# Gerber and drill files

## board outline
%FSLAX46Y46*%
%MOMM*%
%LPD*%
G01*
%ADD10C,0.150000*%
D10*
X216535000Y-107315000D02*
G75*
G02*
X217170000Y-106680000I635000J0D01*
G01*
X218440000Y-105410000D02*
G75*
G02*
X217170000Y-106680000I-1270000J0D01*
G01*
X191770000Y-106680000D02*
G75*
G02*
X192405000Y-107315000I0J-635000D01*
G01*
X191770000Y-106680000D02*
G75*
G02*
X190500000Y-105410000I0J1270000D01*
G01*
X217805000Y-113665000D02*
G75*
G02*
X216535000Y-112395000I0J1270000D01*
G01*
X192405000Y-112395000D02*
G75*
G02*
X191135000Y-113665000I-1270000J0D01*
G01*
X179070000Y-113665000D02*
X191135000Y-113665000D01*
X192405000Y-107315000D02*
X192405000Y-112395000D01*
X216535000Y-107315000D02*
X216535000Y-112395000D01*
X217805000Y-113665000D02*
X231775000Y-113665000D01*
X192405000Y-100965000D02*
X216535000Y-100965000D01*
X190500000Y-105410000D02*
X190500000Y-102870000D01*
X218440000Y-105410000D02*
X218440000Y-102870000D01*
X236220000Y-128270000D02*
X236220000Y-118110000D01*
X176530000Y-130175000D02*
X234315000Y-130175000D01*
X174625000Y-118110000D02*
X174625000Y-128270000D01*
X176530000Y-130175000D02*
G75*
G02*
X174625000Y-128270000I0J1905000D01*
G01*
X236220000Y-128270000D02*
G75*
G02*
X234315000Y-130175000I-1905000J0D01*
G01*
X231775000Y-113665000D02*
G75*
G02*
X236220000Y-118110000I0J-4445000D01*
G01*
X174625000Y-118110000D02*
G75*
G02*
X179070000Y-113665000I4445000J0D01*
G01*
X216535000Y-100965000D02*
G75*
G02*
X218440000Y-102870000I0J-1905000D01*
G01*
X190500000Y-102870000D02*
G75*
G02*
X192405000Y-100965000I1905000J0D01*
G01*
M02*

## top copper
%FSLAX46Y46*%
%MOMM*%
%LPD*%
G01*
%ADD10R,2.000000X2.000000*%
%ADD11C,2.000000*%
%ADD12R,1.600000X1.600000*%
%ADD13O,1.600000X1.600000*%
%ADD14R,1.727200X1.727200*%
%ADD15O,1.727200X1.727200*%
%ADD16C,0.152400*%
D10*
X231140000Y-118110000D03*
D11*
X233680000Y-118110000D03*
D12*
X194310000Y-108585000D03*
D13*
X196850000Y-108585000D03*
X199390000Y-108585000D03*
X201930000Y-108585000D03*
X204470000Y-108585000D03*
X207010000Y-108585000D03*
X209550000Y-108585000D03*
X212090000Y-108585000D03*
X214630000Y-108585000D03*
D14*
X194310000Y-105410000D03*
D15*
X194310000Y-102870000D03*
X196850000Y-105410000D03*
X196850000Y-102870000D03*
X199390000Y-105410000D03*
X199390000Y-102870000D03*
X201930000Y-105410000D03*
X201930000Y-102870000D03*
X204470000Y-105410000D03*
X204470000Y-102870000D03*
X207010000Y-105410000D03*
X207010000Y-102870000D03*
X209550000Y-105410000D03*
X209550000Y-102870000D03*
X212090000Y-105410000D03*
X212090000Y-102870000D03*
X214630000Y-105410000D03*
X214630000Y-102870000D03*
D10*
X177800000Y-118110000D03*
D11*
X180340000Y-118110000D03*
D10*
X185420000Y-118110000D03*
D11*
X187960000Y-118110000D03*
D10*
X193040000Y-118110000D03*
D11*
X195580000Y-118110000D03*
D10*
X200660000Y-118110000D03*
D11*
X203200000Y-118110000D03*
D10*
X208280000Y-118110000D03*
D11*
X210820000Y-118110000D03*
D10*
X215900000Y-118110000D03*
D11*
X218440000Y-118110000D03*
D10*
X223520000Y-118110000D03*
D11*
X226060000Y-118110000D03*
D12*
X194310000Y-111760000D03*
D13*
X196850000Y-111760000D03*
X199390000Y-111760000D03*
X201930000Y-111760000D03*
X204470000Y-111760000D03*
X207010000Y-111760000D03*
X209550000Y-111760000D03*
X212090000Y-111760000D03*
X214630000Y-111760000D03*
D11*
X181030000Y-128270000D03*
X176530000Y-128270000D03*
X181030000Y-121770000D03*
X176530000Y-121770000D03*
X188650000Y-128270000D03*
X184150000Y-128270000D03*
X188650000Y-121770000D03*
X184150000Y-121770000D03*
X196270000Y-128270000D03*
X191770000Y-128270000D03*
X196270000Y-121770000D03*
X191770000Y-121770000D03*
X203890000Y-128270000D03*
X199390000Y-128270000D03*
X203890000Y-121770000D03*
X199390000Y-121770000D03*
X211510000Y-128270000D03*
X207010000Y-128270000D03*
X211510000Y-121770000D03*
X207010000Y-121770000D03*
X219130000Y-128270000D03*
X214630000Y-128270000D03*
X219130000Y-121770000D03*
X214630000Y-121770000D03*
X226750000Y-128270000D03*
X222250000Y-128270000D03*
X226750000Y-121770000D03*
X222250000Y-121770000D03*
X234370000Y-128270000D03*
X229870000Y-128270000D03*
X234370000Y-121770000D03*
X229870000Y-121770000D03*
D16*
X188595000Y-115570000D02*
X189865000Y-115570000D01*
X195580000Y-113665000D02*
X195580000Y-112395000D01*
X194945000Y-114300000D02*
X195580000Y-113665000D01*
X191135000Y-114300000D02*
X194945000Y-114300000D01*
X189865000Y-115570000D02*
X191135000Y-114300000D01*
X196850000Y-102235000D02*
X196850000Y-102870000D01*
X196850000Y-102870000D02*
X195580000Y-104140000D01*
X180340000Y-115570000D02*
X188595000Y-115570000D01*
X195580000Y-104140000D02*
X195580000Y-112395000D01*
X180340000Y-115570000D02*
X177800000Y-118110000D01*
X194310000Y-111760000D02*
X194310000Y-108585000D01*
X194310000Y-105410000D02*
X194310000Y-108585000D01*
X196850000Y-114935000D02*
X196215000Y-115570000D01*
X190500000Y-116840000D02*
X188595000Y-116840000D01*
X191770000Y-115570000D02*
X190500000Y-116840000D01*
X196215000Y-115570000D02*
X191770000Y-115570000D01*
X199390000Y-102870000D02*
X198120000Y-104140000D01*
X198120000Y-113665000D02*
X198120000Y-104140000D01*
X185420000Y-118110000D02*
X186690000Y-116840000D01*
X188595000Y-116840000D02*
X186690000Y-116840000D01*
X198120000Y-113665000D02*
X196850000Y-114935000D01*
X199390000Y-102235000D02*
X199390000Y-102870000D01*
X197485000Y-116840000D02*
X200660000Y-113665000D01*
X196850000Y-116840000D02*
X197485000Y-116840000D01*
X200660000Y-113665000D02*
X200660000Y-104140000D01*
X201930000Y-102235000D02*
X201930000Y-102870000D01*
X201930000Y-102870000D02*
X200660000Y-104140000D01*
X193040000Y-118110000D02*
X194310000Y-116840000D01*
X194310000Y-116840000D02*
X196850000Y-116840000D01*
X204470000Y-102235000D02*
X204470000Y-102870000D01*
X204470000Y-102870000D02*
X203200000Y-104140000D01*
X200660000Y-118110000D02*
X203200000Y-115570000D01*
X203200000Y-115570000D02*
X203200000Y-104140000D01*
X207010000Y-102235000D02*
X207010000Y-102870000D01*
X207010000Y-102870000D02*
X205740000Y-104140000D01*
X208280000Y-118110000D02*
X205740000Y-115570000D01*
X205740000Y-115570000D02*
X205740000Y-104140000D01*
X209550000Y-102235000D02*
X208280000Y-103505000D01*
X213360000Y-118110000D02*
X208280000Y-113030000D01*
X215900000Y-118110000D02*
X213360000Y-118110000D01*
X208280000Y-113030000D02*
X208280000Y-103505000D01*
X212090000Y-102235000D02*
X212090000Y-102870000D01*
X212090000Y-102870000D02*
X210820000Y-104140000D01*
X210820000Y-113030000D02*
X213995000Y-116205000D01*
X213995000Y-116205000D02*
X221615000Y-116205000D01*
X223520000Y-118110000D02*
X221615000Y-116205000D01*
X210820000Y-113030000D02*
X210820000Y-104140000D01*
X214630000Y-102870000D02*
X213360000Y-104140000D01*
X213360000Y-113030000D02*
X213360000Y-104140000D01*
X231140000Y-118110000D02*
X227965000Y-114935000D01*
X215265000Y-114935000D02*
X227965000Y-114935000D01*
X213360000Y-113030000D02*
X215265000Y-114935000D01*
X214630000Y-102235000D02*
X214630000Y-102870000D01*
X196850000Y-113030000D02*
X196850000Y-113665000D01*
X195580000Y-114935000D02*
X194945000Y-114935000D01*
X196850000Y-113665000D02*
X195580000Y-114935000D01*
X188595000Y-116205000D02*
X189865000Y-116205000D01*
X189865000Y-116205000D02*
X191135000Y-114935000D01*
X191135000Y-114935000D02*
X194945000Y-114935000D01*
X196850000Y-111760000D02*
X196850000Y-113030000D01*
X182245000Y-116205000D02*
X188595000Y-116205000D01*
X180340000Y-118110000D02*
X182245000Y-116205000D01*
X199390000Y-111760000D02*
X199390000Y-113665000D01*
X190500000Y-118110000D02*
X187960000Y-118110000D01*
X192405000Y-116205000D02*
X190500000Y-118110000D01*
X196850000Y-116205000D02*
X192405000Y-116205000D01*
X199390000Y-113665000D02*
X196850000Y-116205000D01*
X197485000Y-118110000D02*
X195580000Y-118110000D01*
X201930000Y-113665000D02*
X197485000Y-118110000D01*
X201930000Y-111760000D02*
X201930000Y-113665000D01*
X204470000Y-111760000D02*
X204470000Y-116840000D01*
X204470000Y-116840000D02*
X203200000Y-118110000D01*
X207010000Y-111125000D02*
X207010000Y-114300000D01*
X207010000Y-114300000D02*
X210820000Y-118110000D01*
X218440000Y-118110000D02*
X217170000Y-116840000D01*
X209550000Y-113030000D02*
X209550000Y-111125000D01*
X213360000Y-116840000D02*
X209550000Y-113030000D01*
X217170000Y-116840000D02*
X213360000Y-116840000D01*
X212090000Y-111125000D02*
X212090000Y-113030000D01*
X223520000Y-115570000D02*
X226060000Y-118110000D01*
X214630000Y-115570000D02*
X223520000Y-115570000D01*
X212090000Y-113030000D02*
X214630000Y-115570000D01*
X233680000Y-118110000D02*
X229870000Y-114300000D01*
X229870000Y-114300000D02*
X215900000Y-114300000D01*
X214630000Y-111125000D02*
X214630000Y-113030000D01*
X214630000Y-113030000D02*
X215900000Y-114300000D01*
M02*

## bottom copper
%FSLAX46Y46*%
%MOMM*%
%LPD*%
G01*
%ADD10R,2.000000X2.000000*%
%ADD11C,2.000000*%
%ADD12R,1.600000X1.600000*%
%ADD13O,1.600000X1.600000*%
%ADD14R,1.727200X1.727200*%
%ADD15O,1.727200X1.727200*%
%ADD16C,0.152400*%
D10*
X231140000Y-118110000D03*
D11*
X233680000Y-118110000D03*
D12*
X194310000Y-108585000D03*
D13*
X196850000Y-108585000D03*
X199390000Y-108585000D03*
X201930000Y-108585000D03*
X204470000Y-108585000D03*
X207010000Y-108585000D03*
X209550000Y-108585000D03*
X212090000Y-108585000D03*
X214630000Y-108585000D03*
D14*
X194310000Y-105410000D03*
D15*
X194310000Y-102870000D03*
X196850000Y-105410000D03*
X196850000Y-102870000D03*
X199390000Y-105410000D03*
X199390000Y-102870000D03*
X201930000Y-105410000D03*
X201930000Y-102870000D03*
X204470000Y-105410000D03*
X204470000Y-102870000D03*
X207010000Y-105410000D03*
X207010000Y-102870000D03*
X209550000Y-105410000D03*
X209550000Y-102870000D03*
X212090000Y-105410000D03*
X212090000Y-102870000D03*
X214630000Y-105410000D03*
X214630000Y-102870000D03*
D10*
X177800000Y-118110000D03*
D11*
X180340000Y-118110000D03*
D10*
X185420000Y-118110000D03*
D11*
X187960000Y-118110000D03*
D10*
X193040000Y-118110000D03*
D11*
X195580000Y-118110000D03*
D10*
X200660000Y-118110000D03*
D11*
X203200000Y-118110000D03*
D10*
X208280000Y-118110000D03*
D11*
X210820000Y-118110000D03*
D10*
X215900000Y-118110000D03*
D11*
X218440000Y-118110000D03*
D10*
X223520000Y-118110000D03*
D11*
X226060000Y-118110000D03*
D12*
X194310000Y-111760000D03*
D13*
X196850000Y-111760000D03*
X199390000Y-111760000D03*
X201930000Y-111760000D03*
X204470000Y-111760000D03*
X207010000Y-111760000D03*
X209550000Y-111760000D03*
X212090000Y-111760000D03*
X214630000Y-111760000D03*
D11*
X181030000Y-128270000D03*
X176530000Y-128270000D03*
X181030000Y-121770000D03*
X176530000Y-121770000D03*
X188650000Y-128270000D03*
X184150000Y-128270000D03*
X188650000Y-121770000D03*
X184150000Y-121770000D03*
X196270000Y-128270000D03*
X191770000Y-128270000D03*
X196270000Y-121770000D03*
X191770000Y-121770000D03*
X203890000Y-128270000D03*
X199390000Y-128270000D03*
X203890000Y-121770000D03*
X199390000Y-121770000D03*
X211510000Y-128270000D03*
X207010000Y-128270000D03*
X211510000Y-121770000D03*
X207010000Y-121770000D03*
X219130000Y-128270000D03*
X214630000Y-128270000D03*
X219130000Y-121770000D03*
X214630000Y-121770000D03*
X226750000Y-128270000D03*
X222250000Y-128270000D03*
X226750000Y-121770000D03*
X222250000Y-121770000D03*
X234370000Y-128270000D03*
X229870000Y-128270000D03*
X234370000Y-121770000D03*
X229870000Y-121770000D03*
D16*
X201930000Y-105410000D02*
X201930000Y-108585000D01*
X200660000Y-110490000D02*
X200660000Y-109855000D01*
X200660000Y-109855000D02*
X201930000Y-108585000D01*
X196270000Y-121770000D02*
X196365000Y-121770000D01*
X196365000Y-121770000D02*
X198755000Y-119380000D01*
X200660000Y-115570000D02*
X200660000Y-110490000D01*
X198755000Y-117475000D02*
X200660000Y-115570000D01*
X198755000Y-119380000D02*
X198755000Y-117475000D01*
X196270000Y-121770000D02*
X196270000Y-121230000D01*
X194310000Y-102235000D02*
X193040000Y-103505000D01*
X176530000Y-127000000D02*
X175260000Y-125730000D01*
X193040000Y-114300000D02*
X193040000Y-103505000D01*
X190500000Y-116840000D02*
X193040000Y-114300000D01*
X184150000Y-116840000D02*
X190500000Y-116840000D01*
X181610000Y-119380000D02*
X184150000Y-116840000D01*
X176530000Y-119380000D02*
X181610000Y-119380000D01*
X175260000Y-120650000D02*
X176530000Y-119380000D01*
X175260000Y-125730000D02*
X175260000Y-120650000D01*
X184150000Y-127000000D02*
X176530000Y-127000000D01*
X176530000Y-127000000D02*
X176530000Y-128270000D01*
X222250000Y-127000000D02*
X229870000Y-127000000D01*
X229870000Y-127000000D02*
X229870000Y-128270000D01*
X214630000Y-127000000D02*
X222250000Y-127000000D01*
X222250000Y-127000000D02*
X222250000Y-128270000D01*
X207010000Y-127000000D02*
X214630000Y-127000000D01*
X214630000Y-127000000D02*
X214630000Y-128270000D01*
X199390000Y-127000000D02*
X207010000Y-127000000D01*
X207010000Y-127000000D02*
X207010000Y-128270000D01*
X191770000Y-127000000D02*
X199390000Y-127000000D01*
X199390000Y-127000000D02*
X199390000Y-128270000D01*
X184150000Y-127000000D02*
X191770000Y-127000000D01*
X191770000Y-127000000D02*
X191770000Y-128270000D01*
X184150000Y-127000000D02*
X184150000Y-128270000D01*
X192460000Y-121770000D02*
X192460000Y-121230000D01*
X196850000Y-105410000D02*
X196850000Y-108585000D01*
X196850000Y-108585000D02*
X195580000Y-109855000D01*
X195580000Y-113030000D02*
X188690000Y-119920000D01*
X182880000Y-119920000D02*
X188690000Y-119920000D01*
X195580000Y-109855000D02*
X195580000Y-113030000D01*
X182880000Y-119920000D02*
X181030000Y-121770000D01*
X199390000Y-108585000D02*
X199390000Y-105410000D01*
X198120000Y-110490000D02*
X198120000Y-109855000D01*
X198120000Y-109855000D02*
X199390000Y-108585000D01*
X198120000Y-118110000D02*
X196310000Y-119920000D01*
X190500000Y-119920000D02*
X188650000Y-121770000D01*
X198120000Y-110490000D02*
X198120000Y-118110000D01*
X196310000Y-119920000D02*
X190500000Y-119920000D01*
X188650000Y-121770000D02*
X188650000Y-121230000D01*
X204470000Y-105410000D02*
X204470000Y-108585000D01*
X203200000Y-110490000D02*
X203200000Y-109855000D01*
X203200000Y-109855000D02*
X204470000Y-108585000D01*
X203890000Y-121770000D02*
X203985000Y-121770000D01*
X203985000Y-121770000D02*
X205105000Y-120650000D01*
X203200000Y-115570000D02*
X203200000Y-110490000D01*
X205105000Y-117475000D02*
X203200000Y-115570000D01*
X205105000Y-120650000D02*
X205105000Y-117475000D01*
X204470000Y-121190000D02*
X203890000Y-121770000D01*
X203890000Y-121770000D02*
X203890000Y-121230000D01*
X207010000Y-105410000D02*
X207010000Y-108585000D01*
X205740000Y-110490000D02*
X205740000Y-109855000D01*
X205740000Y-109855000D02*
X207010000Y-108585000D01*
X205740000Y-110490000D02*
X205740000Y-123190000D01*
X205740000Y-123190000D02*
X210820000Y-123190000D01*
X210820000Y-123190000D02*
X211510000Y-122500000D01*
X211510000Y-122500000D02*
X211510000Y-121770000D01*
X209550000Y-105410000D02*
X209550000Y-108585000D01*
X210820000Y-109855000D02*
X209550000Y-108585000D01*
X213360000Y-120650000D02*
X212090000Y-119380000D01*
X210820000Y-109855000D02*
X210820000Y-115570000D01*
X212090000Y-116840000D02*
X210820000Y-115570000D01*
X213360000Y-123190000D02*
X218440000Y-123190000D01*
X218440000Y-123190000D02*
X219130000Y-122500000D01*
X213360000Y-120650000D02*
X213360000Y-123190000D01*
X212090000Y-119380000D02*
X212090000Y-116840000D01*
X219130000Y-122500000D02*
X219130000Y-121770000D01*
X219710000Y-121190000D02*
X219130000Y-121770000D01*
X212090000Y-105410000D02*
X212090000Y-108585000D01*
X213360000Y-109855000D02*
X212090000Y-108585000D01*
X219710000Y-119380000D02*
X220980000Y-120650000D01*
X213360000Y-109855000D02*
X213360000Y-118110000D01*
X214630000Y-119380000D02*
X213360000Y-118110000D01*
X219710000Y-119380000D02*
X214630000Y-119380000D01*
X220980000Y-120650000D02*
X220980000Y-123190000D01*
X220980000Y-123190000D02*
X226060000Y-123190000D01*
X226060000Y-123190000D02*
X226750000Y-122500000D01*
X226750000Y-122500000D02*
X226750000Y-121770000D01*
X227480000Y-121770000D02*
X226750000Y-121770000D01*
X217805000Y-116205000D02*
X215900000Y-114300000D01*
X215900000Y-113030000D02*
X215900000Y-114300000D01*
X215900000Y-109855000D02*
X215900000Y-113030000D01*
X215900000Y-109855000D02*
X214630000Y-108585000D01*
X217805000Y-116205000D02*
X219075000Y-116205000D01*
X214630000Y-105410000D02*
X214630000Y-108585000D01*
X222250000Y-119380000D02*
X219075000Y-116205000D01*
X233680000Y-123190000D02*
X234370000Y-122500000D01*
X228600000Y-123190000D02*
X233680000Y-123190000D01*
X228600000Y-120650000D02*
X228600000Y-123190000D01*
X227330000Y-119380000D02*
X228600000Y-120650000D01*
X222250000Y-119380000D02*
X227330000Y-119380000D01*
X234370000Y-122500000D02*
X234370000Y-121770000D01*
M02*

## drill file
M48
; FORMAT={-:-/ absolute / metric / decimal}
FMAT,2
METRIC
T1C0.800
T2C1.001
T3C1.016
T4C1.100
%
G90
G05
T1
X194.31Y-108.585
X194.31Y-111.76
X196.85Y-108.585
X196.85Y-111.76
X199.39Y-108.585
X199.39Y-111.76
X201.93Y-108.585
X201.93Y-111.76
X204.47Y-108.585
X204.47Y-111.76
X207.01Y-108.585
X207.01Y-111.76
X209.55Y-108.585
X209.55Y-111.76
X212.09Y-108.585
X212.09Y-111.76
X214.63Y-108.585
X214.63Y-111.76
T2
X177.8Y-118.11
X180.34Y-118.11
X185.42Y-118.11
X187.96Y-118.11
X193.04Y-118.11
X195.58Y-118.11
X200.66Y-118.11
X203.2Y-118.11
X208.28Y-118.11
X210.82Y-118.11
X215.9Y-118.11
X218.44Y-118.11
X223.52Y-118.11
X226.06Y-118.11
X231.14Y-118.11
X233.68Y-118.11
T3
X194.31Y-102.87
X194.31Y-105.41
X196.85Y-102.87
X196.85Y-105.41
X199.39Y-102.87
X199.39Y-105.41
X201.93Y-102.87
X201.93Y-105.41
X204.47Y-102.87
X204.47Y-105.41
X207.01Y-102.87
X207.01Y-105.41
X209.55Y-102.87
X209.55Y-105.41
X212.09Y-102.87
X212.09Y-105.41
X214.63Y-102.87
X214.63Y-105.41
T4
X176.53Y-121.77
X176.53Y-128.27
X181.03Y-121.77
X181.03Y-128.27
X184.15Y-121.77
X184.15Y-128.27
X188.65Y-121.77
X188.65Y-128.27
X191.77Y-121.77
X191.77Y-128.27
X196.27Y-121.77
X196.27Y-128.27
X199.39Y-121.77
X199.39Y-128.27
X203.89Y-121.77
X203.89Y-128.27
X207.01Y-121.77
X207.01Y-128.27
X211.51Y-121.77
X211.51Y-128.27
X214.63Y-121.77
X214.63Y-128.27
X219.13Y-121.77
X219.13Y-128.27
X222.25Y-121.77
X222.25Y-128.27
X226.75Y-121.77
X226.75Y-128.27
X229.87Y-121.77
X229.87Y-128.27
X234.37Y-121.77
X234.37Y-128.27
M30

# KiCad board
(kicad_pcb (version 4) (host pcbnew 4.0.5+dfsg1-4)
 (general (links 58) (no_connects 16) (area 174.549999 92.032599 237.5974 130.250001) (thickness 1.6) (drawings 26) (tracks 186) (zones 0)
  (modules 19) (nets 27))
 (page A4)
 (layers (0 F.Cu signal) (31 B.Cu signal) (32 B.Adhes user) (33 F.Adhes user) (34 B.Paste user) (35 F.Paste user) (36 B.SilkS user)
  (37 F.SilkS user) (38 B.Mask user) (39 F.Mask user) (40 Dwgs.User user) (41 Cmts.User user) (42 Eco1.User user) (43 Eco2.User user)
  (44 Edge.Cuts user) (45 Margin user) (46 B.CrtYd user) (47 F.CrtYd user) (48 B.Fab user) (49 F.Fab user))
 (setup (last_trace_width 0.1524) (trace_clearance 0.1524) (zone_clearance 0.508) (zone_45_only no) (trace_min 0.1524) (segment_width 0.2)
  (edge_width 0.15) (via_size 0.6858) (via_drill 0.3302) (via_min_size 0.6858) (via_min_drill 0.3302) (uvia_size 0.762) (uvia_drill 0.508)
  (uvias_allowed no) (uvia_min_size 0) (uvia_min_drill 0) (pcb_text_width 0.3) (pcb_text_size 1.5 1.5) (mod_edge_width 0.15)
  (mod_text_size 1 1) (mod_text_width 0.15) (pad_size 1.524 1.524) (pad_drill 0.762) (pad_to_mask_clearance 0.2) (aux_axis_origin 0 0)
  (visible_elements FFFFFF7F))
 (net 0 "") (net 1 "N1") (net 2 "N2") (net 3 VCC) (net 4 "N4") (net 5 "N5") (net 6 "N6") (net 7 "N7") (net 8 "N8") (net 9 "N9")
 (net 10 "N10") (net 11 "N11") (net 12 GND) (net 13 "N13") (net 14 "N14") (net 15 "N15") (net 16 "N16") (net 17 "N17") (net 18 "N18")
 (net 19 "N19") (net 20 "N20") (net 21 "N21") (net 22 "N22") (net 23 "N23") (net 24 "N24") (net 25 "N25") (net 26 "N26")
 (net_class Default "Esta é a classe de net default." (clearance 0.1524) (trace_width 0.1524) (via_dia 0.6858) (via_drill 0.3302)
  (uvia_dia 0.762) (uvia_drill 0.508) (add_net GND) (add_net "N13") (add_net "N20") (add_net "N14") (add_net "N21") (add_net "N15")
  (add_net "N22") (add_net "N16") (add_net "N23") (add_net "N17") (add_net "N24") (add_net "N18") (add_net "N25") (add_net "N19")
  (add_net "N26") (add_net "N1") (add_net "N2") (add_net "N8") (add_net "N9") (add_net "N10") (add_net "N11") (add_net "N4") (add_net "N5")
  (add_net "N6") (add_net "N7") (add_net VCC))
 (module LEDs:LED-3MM (layer F.Cu) (at 231.14 118.11)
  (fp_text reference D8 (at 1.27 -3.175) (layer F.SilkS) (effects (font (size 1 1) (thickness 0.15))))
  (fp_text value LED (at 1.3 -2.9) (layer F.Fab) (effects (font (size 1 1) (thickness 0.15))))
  (pad 1 thru_hole rect (at 0 0 90) (size 2 2) (drill 1.00076) (layers *.Cu *.Mask) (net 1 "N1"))
  (pad 2 thru_hole circle (at 2.54 0) (size 2 2) (drill 1.00076) (layers *.Cu *.Mask) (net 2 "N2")))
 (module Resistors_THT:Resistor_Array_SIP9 (layer F.Cu) (at 194.31 108.585)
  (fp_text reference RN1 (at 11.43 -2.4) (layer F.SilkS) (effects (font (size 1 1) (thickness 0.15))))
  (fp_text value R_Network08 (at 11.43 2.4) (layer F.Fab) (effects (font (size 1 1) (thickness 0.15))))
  (pad 1 thru_hole rect (at 0 0) (size 1.6 1.6) (drill 0.8) (layers *.Cu *.Mask) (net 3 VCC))
  (pad 2 thru_hole oval (at 2.54 0) (size 1.6 1.6) (drill 0.8) (layers *.Cu *.Mask) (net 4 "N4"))
  (pad 3 thru_hole oval (at 5.08 0) (size 1.6 1.6) (drill 0.8) (layers *.Cu *.Mask) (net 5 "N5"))
  (pad 4 thru_hole oval (at 7.62 0) (size 1.6 1.6) (drill 0.8) (layers *.Cu *.Mask) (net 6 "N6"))
  (pad 5 thru_hole oval (at 10.16 0) (size 1.6 1.6) (drill 0.8) (layers *.Cu *.Mask) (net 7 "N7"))
  (pad 6 thru_hole oval (at 12.7 0) (size 1.6 1.6) (drill 0.8) (layers *.Cu *.Mask) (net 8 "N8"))
  (pad 7 thru_hole oval (at 15.24 0) (size 1.6 1.6) (drill 0.8) (layers *.Cu *.Mask) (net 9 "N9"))
  (pad 8 thru_hole oval (at 17.78 0) (size 1.6 1.6) (drill 0.8) (layers *.Cu *.Mask) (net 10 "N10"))
  (pad 9 thru_hole oval (at 20.32 0) (size 1.6 1.6) (drill 0.8) (layers *.Cu *.Mask) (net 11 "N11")))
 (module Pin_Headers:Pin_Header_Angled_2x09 (layer F.Cu) (at 194.31 105.41 90)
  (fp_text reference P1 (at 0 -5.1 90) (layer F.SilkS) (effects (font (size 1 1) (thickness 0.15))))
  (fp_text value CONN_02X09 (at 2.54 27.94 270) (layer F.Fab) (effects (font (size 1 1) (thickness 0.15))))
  (pad 1 thru_hole rect (at 0 0 90) (size 1.7272 1.7272) (drill 1.016) (layers *.Cu *.Mask) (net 3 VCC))
  (pad 2 thru_hole oval (at 2.54 0 90) (size 1.7272 1.7272) (drill 1.016) (layers *.Cu *.Mask) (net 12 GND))
  (pad 3 thru_hole oval (at 0 2.54 90) (size 1.7272 1.7272) (drill 1.016) (layers *.Cu *.Mask) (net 4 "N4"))
  (pad 4 thru_hole oval (at 2.54 2.54 90) (size 1.7272 1.7272) (drill 1.016) (layers *.Cu *.Mask) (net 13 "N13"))
  (pad 5 thru_hole oval (at 0 5.08 90) (size 1.7272 1.7272) (drill 1.016) (layers *.Cu *.Mask) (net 5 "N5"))
  (pad 6 thru_hole oval (at 2.54 5.08 90) (size 1.7272 1.7272) (drill 1.016) (layers *.Cu *.Mask) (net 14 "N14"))
  (pad 7 thru_hole oval (at 0 7.62 90) (size 1.7272 1.7272) (drill 1.016) (layers *.Cu *.Mask) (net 6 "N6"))
  (pad 8 thru_hole oval (at 2.54 7.62 90) (size 1.7272 1.7272) (drill 1.016) (layers *.Cu *.Mask) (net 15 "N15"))
  (pad 9 thru_hole oval (at 0 10.16 90) (size 1.7272 1.7272) (drill 1.016) (layers *.Cu *.Mask) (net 7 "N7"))
  (pad 10 thru_hole oval (at 2.54 10.16 90) (size 1.7272 1.7272) (drill 1.016) (layers *.Cu *.Mask) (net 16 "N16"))
  (pad 11 thru_hole oval (at 0 12.7 90) (size 1.7272 1.7272) (drill 1.016) (layers *.Cu *.Mask) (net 8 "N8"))
  (pad 12 thru_hole oval (at 2.54 12.7 90) (size 1.7272 1.7272) (drill 1.016) (layers *.Cu *.Mask) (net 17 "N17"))
  (pad 13 thru_hole oval (at 0 15.24 90) (size 1.7272 1.7272) (drill 1.016) (layers *.Cu *.Mask) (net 9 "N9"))
  (pad 14 thru_hole oval (at 2.54 15.24 90) (size 1.7272 1.7272) (drill 1.016) (layers *.Cu *.Mask) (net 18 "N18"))
  (pad 15 thru_hole oval (at 0 17.78 90) (size 1.7272 1.7272) (drill 1.016) (layers *.Cu *.Mask) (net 10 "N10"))
  (pad 16 thru_hole oval (at 2.54 17.78 90) (size 1.7272 1.7272) (drill 1.016) (layers *.Cu *.Mask) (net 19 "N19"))
  (pad 17 thru_hole oval (at 0 20.32 90) (size 1.7272 1.7272) (drill 1.016) (layers *.Cu *.Mask) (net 11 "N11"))
  (pad 18 thru_hole oval (at 2.54 20.32 90) (size 1.7272 1.7272) (drill 1.016) (layers *.Cu *.Mask) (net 1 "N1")))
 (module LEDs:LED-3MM (layer F.Cu) (at 177.8 118.11)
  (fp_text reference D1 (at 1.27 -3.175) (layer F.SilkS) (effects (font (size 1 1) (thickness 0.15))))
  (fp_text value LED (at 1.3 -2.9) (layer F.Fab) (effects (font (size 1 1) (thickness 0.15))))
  (pad 1 thru_hole rect (at 0 0 90) (size 2 2) (drill 1.00076) (layers *.Cu *.Mask) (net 13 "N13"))
  (pad 2 thru_hole circle (at 2.54 0) (size 2 2) (drill 1.00076) (layers *.Cu *.Mask) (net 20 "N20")))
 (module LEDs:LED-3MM (layer F.Cu) (at 185.42 118.11)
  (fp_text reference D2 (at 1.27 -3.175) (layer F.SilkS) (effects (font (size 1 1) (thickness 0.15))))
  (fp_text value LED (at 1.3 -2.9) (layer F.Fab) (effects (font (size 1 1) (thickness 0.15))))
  (pad 1 thru_hole rect (at 0 0 90) (size 2 2) (drill 1.00076) (layers *.Cu *.Mask) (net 14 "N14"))
  (pad 2 thru_hole circle (at 2.54 0) (size 2 2) (drill 1.00076) (layers *.Cu *.Mask) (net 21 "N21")))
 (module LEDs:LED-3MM (layer F.Cu) (at 193.04 118.11)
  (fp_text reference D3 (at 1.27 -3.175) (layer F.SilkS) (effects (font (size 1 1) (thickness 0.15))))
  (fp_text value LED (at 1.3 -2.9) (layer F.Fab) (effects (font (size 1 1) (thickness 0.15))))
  (pad 1 thru_hole rect (at 0 0 90) (size 2 2) (drill 1.00076) (layers *.Cu *.Mask) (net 15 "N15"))
  (pad 2 thru_hole circle (at 2.54 0) (size 2 2) (drill 1.00076) (layers *.Cu *.Mask) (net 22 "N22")))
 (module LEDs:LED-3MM (layer F.Cu) (at 200.66 118.11)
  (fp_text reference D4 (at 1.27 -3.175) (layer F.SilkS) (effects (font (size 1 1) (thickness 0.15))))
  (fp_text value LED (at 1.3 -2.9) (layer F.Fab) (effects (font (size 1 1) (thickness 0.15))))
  (pad 1 thru_hole rect (at 0 0 90) (size 2 2) (drill 1.00076) (layers *.Cu *.Mask) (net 16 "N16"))
  (pad 2 thru_hole circle (at 2.54 0) (size 2 2) (drill 1.00076) (layers *.Cu *.Mask) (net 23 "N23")))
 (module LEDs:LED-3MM (layer F.Cu) (at 208.28 118.11)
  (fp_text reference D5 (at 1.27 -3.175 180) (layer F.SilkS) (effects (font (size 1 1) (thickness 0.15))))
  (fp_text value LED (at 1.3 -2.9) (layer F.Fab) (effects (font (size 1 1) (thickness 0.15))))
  (pad 1 thru_hole rect (at 0 0 90) (size 2 2) (drill 1.00076) (layers *.Cu *.Mask) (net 17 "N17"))
  (pad 2 thru_hole circle (at 2.54 0) (size 2 2) (drill 1.00076) (layers *.Cu *.Mask) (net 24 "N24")))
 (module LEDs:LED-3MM (layer F.Cu) (at 215.9 118.11)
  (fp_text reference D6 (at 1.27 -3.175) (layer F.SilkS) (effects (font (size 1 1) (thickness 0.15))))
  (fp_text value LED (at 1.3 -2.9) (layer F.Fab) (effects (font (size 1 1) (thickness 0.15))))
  (pad 1 thru_hole rect (at 0 0 90) (size 2 2) (drill 1.00076) (layers *.Cu *.Mask) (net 18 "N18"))
  (pad 2 thru_hole circle (at 2.54 0) (size 2 2) (drill 1.00076) (layers *.Cu *.Mask) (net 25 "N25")))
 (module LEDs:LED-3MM (layer F.Cu) (at 223.52 118.11)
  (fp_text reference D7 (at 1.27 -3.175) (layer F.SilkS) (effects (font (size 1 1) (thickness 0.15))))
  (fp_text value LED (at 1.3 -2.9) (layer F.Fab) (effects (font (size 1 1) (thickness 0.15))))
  (pad 1 thru_hole rect (at 0 0 90) (size 2 2) (drill 1.00076) (layers *.Cu *.Mask) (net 19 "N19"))
  (pad 2 thru_hole circle (at 2.54 0) (size 2 2) (drill 1.00076) (layers *.Cu *.Mask) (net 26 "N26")))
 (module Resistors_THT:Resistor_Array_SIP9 (layer F.Cu) (at 194.31 111.76)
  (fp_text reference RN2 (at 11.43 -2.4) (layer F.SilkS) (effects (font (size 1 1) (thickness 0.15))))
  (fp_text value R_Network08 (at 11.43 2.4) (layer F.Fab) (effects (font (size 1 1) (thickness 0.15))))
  (pad 1 thru_hole rect (at 0 0) (size 1.6 1.6) (drill 0.8) (layers *.Cu *.Mask) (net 3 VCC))
  (pad 2 thru_hole oval (at 2.54 0) (size 1.6 1.6) (drill 0.8) (layers *.Cu *.Mask) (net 20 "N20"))
  (pad 3 thru_hole oval (at 5.08 0) (size 1.6 1.6) (drill 0.8) (layers *.Cu *.Mask) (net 21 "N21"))
  (pad 4 thru_hole oval (at 7.62 0) (size 1.6 1.6) (drill 0.8) (layers *.Cu *.Mask) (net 22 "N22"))
  (pad 5 thru_hole oval (at 10.16 0) (size 1.6 1.6) (drill 0.8) (layers *.Cu *.Mask) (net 23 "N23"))
  (pad 6 thru_hole oval (at 12.7 0) (size 1.6 1.6) (drill 0.8) (layers *.Cu *.Mask) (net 24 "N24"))
  (pad 7 thru_hole oval (at 15.24 0) (size 1.6 1.6) (drill 0.8) (layers *.Cu *.Mask) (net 25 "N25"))
  (pad 8 thru_hole oval (at 17.78 0) (size 1.6 1.6) (drill 0.8) (layers *.Cu *.Mask) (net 26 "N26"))
  (pad 9 thru_hole oval (at 20.32 0) (size 1.6 1.6) (drill 0.8) (layers *.Cu *.Mask) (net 2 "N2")))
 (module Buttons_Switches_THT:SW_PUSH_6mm (layer F.Cu) (at 176.53 128.27 90)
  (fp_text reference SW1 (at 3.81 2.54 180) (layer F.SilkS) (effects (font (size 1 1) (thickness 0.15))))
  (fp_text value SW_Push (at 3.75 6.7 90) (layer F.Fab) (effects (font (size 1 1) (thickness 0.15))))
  (pad 2 thru_hole circle (at 0 4.5 180) (size 2 2) (drill 1.1) (layers *.Cu *.Mask) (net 4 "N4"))
  (pad 1 thru_hole circle (at 0 0 180) (size 2 2) (drill 1.1) (layers *.Cu *.Mask) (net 12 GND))
  (pad 2 thru_hole circle (at 6.5 4.5 180) (size 2 2) (drill 1.1) (layers *.Cu *.Mask) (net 4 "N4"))
  (pad 1 thru_hole circle (at 6.5 0 180) (size 2 2) (drill 1.1) (layers *.Cu *.Mask) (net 12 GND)))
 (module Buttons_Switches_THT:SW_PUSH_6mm (layer F.Cu) (at 184.15 128.27 90)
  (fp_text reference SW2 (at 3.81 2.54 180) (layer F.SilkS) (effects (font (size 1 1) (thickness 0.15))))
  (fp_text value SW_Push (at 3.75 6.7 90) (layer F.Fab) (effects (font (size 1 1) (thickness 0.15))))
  (pad 2 thru_hole circle (at 0 4.5 180) (size 2 2) (drill 1.1) (layers *.Cu *.Mask) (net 5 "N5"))
  (pad 1 thru_hole circle (at 0 0 180) (size 2 2) (drill 1.1) (layers *.Cu *.Mask) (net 12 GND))
  (pad 2 thru_hole circle (at 6.5 4.5 180) (size 2 2) (drill 1.1) (layers *.Cu *.Mask) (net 5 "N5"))
  (pad 1 thru_hole circle (at 6.5 0 180) (size 2 2) (drill 1.1) (layers *.Cu *.Mask) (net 12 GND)))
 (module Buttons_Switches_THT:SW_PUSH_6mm (layer F.Cu) (at 191.77 128.27 90)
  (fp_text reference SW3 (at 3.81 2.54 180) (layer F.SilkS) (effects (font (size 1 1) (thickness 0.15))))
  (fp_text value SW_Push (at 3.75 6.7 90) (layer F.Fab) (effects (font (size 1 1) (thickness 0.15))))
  (pad 2 thru_hole circle (at 0 4.5 180) (size 2 2) (drill 1.1) (layers *.Cu *.Mask) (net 6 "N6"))
  (pad 1 thru_hole circle (at 0 0 180) (size 2 2) (drill 1.1) (layers *.Cu *.Mask) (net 12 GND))
  (pad 2 thru_hole circle (at 6.5 4.5 180) (size 2 2) (drill 1.1) (layers *.Cu *.Mask) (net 6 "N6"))
  (pad 1 thru_hole circle (at 6.5 0 180) (size 2 2) (drill 1.1) (layers *.Cu *.Mask) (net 12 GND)))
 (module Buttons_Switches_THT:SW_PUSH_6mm (layer F.Cu) (at 199.39 128.27 90)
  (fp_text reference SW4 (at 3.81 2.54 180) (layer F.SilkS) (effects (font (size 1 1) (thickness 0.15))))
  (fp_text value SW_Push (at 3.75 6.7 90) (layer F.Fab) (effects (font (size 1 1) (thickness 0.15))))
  (pad 2 thru_hole circle (at 0 4.5 180) (size 2 2) (drill 1.1) (layers *.Cu *.Mask) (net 7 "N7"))
  (pad 1 thru_hole circle (at 0 0 180) (size 2 2) (drill 1.1) (layers *.Cu *.Mask) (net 12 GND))
  (pad 2 thru_hole circle (at 6.5 4.5 180) (size 2 2) (drill 1.1) (layers *.Cu *.Mask) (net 7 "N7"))
  (pad 1 thru_hole circle (at 6.5 0 180) (size 2 2) (drill 1.1) (layers *.Cu *.Mask) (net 12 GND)))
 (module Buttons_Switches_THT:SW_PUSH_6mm (layer F.Cu) (at 207.01 128.27 90)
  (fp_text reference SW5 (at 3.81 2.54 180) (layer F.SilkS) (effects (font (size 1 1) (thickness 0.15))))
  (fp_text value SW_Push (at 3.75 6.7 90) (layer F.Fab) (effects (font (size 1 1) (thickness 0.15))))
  (pad 2 thru_hole circle (at 0 4.5 180) (size 2 2) (drill 1.1) (layers *.Cu *.Mask) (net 8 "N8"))
  (pad 1 thru_hole circle (at 0 0 180) (size 2 2) (drill 1.1) (layers *.Cu *.Mask) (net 12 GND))
  (pad 2 thru_hole circle (at 6.5 4.5 180) (size 2 2) (drill 1.1) (layers *.Cu *.Mask) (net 8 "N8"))
  (pad 1 thru_hole circle (at 6.5 0 180) (size 2 2) (drill 1.1) (layers *.Cu *.Mask) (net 12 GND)))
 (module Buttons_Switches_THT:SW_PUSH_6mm (layer F.Cu) (at 214.63 128.27 90)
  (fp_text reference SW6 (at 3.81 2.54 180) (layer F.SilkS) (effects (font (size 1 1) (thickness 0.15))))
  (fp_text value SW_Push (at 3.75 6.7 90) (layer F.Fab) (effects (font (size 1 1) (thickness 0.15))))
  (pad 2 thru_hole circle (at 0 4.5 180) (size 2 2) (drill 1.1) (layers *.Cu *.Mask) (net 9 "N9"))
  (pad 1 thru_hole circle (at 0 0 180) (size 2 2) (drill 1.1) (layers *.Cu *.Mask) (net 12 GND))
  (pad 2 thru_hole circle (at 6.5 4.5 180) (size 2 2) (drill 1.1) (layers *.Cu *.Mask) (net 9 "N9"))
  (pad 1 thru_hole circle (at 6.5 0 180) (size 2 2) (drill 1.1) (layers *.Cu *.Mask) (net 12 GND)))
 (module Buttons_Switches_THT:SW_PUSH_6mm (layer F.Cu) (at 222.25 128.27 90)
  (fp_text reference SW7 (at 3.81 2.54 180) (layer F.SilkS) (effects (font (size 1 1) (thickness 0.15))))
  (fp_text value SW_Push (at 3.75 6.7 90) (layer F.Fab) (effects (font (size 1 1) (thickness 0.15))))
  (pad 2 thru_hole circle (at 0 4.5 180) (size 2 2) (drill 1.1) (layers *.Cu *.Mask) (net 10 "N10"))
  (pad 1 thru_hole circle (at 0 0 180) (size 2 2) (drill 1.1) (layers *.Cu *.Mask) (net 12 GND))
  (pad 2 thru_hole circle (at 6.5 4.5 180) (size 2 2) (drill 1.1) (layers *.Cu *.Mask) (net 10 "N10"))
  (pad 1 thru_hole circle (at 6.5 0 180) (size 2 2) (drill 1.1) (layers *.Cu *.Mask) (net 12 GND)))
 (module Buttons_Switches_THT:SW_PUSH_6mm (layer F.Cu) (at 229.87 128.27 90)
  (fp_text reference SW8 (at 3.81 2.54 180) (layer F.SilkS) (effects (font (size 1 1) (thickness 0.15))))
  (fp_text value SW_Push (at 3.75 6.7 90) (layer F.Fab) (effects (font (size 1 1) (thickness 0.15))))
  (pad 2 thru_hole circle (at 0 4.5 180) (size 2 2) (drill 1.1) (layers *.Cu *.Mask) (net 11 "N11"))
  (pad 1 thru_hole circle (at 0 0 180) (size 2 2) (drill 1.1) (layers *.Cu *.Mask) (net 12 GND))
  (pad 2 thru_hole circle (at 6.5 4.5 180) (size 2 2) (drill 1.1) (layers *.Cu *.Mask) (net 11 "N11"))
  (pad 1 thru_hole circle (at 6.5 0 180) (size 2 2) (drill 1.1) (layers *.Cu *.Mask) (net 12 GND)))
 (gr_arc (start 217.17 107.315) (end 216.535 107.315) (angle 90) (layer Edge.Cuts) (width 0.15))
 (gr_arc (start 217.17 105.41) (end 218.44 105.41) (angle 90) (layer Edge.Cuts) (width 0.15))
 (gr_arc (start 191.77 107.315) (end 191.77 106.68) (angle 90) (layer Edge.Cuts) (width 0.15))
 (gr_arc (start 191.77 105.41) (end 191.77 106.68) (angle 90) (layer Edge.Cuts) (width 0.15))
 (gr_arc (start 217.805 112.395) (end 217.805 113.665) (angle 90) (layer Edge.Cuts) (width 0.15))
 (gr_arc (start 191.135 112.395) (end 192.405 112.395) (angle 90) (layer Edge.Cuts) (width 0.15))
 (gr_line (start 179.07 113.665) (end 191.135 113.665) (angle 90) (layer Edge.Cuts) (width 0.15))
 (gr_line (start 192.405 107.315) (end 192.405 112.395) (angle 90) (layer Edge.Cuts) (width 0.15))
 (gr_line (start 216.535 107.315) (end 216.535 112.395) (angle 90) (layer Edge.Cuts) (width 0.15))
 (gr_line (start 217.805 113.665) (end 231.775 113.665) (angle 90) (layer Edge.Cuts) (width 0.15))
 (gr_line (start 192.405 100.965) (end 216.535 100.965) (angle 90) (layer Edge.Cuts) (width 0.15))
 (gr_line (start 190.5 105.41) (end 190.5 102.87) (angle 90) (layer Edge.Cuts) (width 0.15))
 (gr_line (start 218.44 105.41) (end 218.44 102.87) (angle 90) (layer Edge.Cuts) (width 0.15))
 (gr_line (start 236.22 128.27) (end 236.22 118.11) (angle 90) (layer Edge.Cuts) (width 0.15))
 (gr_line (start 176.53 130.175) (end 234.315 130.175) (angle 90) (layer Edge.Cuts) (width 0.15))
 (gr_line (start 174.625 118.11) (end 174.625 128.27) (angle 90) (layer Edge.Cuts) (width 0.15))
 (gr_arc (start 176.53 128.27) (end 176.53 130.175) (angle 90) (layer Edge.Cuts) (width 0.15))
 (gr_arc (start 234.315 128.27) (end 236.22 128.27) (angle 90) (layer Edge.Cuts) (width 0.15))
 (gr_arc (start 231.775 118.11) (end 231.775 113.665) (angle 90) (layer Edge.Cuts) (width 0.15))
 (gr_arc (start 179.07 118.11) (end 174.625 118.11) (angle 90) (layer Edge.Cuts) (width 0.15))
 (gr_arc (start 216.535 102.87) (end 216.535 100.965) (angle 90) (layer Edge.Cuts) (width 0.15))
 (gr_arc (start 192.405 102.87) (end 190.5 102.87) (angle 90) (layer Edge.Cuts) (width 0.15))
 (segment (start 188.595 115.57) (end 189.865 115.57) (width 0.1524) (layer F.Cu) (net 13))
 (segment (start 195.58 113.665) (end 195.58 112.395) (width 0.1524) (layer F.Cu) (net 13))
 (segment (start 194.945 114.3) (end 195.58 113.665) (width 0.1524) (layer F.Cu) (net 13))
 (segment (start 191.135 114.3) (end 194.945 114.3) (width 0.1524) (layer F.Cu) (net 13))
 (segment (start 189.865 115.57) (end 191.135 114.3) (width 0.1524) (layer F.Cu) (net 13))
 (segment (start 196.85 102.235) (end 196.85 102.87) (width 0.1524) (layer F.Cu) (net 13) (status 30))
 (segment (start 196.85 102.87) (end 195.58 104.14) (width 0.1524) (layer F.Cu) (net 13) (status 10))
 (segment (start 180.34 115.57) (end 188.595 115.57) (width 0.1524) (layer F.Cu) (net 13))
 (segment (start 195.58 104.14) (end 195.58 112.395) (width 0.1524) (layer F.Cu) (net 13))
 (segment (start 180.34 115.57) (end 177.8 118.11) (width 0.1524) (layer F.Cu) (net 13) (status 20))
 (segment (start 194.31 111.76) (end 194.31 108.585) (width 0.1524) (layer F.Cu) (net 3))
 (segment (start 194.31 105.41) (end 194.31 108.585) (width 0.1524) (layer F.Cu) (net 3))
 (segment (start 196.85 114.935) (end 196.215 115.57) (width 0.1524) (layer F.Cu) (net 14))
 (segment (start 190.5 116.84) (end 188.595 116.84) (width 0.1524) (layer F.Cu) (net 14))
 (segment (start 191.77 115.57) (end 190.5 116.84) (width 0.1524) (layer F.Cu) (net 14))
 (segment (start 196.215 115.57) (end 191.77 115.57) (width 0.1524) (layer F.Cu) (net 14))
 (segment (start 199.39 102.87) (end 198.12 104.14) (width 0.1524) (layer F.Cu) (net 14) (status 10))
 (segment (start 198.12 113.665) (end 198.12 104.14) (width 0.1524) (layer F.Cu) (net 14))
 (segment (start 185.42 118.11) (end 186.69 116.84) (width 0.1524) (layer F.Cu) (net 14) (status 10))
 (segment (start 188.595 116.84) (end 186.69 116.84) (width 0.1524) (layer F.Cu) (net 14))
 (segment (start 198.12 113.665) (end 196.85 114.935) (width 0.1524) (layer F.Cu) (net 14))
 (segment (start 199.39 102.235) (end 199.39 102.87) (width 0.1524) (layer F.Cu) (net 14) (status 30))
 (segment (start 197.485 116.84) (end 200.66 113.665) (width 0.1524) (layer F.Cu) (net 15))
 (segment (start 196.85 116.84) (end 197.485 116.84) (width 0.1524) (layer F.Cu) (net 15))
 (segment (start 200.66 113.665) (end 200.66 104.14) (width 0.1524) (layer F.Cu) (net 15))
 (segment (start 201.93 102.235) (end 201.93 102.87) (width 0.1524) (layer F.Cu) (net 15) (status 30))
 (segment (start 201.93 102.87) (end 200.66 104.14) (width 0.1524) (layer F.Cu) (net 15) (status 10))
 (segment (start 193.04 118.11) (end 194.31 116.84) (width 0.1524) (layer F.Cu) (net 15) (status 10))
 (segment (start 194.31 116.84) (end 196.85 116.84) (width 0.1524) (layer F.Cu) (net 15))
 (segment (start 204.47 102.235) (end 204.47 102.87) (width 0.1524) (layer F.Cu) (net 16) (status 30))
 (segment (start 204.47 102.87) (end 203.2 104.14) (width 0.1524) (layer F.Cu) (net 16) (status 10))
 (segment (start 200.66 118.11) (end 203.2 115.57) (width 0.1524) (layer F.Cu) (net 16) (status 10))
 (segment (start 203.2 115.57) (end 203.2 104.14) (width 0.1524) (layer F.Cu) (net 16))
 (segment (start 207.01 102.235) (end 207.01 102.87) (width 0.1524) (layer F.Cu) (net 17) (status 30))
 (segment (start 207.01 102.87) (end 205.74 104.14) (width 0.1524) (layer F.Cu) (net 17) (status 10))
 (segment (start 208.28 118.11) (end 205.74 115.57) (width 0.1524) (layer F.Cu) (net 17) (status 10))
 (segment (start 205.74 115.57) (end 205.74 104.14) (width 0.1524) (layer F.Cu) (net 17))
 (segment (start 209.55 102.235) (end 208.28 103.505) (width 0.1524) (layer F.Cu) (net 18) (status 10))
 (segment (start 213.36 118.11) (end 208.28 113.03) (width 0.1524) (layer F.Cu) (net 18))
 (segment (start 215.9 118.11) (end 213.36 118.11) (width 0.1524) (layer F.Cu) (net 18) (status 10))
 (segment (start 208.28 113.03) (end 208.28 103.505) (width 0.1524) (layer F.Cu) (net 18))
 (segment (start 212.09 102.235) (end 212.09 102.87) (width 0.1524) (layer F.Cu) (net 19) (status 30))
 (segment (start 212.09 102.87) (end 210.82 104.14) (width 0.1524) (layer F.Cu) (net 19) (status 10))
 (segment (start 210.82 113.03) (end 213.995 116.205) (width 0.1524) (layer F.Cu) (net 19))
 (segment (start 213.995 116.205) (end 221.615 116.205) (width 0.1524) (layer F.Cu) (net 19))
 (segment (start 223.52 118.11) (end 221.615 116.205) (width 0.1524) (layer F.Cu) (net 19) (status 10))
 (segment (start 210.82 113.03) (end 210.82 104.14) (width 0.1524) (layer F.Cu) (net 19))
 (segment (start 214.63 102.87) (end 213.36 104.14) (width 0.1524) (layer F.Cu) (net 1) (status 10))
 (segment (start 213.36 113.03) (end 213.36 104.14) (width 0.1524) (layer F.Cu) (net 1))
 (segment (start 231.14 118.11) (end 227.965 114.935) (width 0.1524) (layer F.Cu) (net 1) (status 10))
 (segment (start 215.265 114.935) (end 227.965 114.935) (width 0.1524) (layer F.Cu) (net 1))
 (segment (start 213.36 113.03) (end 215.265 114.935) (width 0.1524) (layer F.Cu) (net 1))
 (segment (start 214.63 102.235) (end 214.63 102.87) (width 0.1524) (layer F.Cu) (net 1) (status 30))
 (segment (start 201.93 105.41) (end 201.93 108.585) (width 0.1524) (layer B.Cu) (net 6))
 (segment (start 200.66 110.49) (end 200.66 109.855) (width 0.1524) (layer B.Cu) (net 6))
 (segment (start 200.66 109.855) (end 201.93 108.585) (width 0.1524) (layer B.Cu) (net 6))
 (segment (start 196.27 121.77) (end 196.365 121.77) (width 0.1524) (layer B.Cu) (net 6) (status 30))
 (segment (start 196.365 121.77) (end 198.755 119.38) (width 0.1524) (layer B.Cu) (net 6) (status 10))
 (segment (start 200.66 115.57) (end 200.66 110.49) (width 0.1524) (layer B.Cu) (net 6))
 (segment (start 198.755 117.475) (end 200.66 115.57) (width 0.1524) (layer B.Cu) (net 6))
 (segment (start 198.755 119.38) (end 198.755 117.475) (width 0.1524) (layer B.Cu) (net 6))
 (segment (start 196.27 121.77) (end 196.27 121.23) (width 0.1524) (layer B.Cu) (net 6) (status 30))
 (segment (start 194.31 102.235) (end 193.04 103.505) (width 0.1524) (layer B.Cu) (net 12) (status 10))
 (segment (start 176.53 127) (end 175.26 125.73) (width 0.1524) (layer B.Cu) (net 12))
 (segment (start 193.04 114.3) (end 193.04 103.505) (width 0.1524) (layer B.Cu) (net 12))
 (segment (start 190.5 116.84) (end 193.04 114.3) (width 0.1524) (layer B.Cu) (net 12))
 (segment (start 184.15 116.84) (end 190.5 116.84) (width 0.1524) (layer B.Cu) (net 12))
 (segment (start 181.61 119.38) (end 184.15 116.84) (width 0.1524) (layer B.Cu) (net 12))
 (segment (start 176.53 119.38) (end 181.61 119.38) (width 0.1524) (layer B.Cu) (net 12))
 (segment (start 175.26 120.65) (end 176.53 119.38) (width 0.1524) (layer B.Cu) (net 12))
 (segment (start 175.26 125.73) (end 175.26 120.65) (width 0.1524) (layer B.Cu) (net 12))
 (segment (start 184.15 127) (end 176.53 127) (width 0.1524) (layer B.Cu) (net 12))
 (segment (start 176.53 127) (end 176.53 128.27) (width 0.1524) (layer B.Cu) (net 12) (status 20))
 (segment (start 222.25 127) (end 229.87 127) (width 0.1524) (layer B.Cu) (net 12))
 (segment (start 229.87 127) (end 229.87 128.27) (width 0.1524) (layer B.Cu) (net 12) (status 20))
 (segment (start 214.63 127) (end 222.25 127) (width 0.1524) (layer B.Cu) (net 12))
 (segment (start 222.25 127) (end 222.25 128.27) (width 0.1524) (layer B.Cu) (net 12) (status 20))
 (segment (start 207.01 127) (end 214.63 127) (width 0.1524) (layer B.Cu) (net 12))
 (segment (start 214.63 127) (end 214.63 128.27) (width 0.1524) (layer B.Cu) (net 12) (status 20))
 (segment (start 199.39 127) (end 207.01 127) (width 0.1524) (layer B.Cu) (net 12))
 (segment (start 207.01 127) (end 207.01 128.27) (width 0.1524) (layer B.Cu) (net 12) (status 20))
 (segment (start 191.77 127) (end 199.39 127) (width 0.1524) (layer B.Cu) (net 12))
 (segment (start 199.39 127) (end 199.39 128.27) (width 0.1524) (layer B.Cu) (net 12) (status 20))
 (segment (start 184.15 127) (end 191.77 127) (width 0.1524) (layer B.Cu) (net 12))
 (segment (start 191.77 127) (end 191.77 128.27) (width 0.1524) (layer B.Cu) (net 12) (status 20))
 (segment (start 184.15 127) (end 184.15 128.27) (width 0.1524) (layer B.Cu) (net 12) (status 20))
 (segment (start 192.46 121.77) (end 192.46 121.23) (width 0.1524) (layer B.Cu) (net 12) (status 30))
 (segment (start 196.85 105.41) (end 196.85 108.585) (width 0.1524) (layer B.Cu) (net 4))
 (segment (start 196.85 108.585) (end 195.58 109.855) (width 0.1524) (layer B.Cu) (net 4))
 (segment (start 195.58 113.03) (end 188.69 119.92) (width 0.1524) (layer B.Cu) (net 4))
 (segment (start 182.88 119.92) (end 188.69 119.92) (width 0.1524) (layer B.Cu) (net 4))
 (segment (start 195.58 109.855) (end 195.58 113.03) (width 0.1524) (layer B.Cu) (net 4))
 (segment (start 182.88 119.92) (end 181.03 121.77) (width 0.1524) (layer B.Cu) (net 4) (status 20))
 (segment (start 199.39 108.585) (end 199.39 105.41) (width 0.1524) (layer B.Cu) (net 5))
 (segment (start 198.12 110.49) (end 198.12 109.855) (width 0.1524) (layer B.Cu) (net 5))
 (segment (start 198.12 109.855) (end 199.39 108.585) (width 0.1524) (layer B.Cu) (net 5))
 (segment (start 198.12 118.11) (end 196.31 119.92) (width 0.1524) (layer B.Cu) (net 5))
 (segment (start 190.5 119.92) (end 188.65 121.77) (width 0.1524) (layer B.Cu) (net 5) (status 20))
 (segment (start 198.12 110.49) (end 198.12 118.11) (width 0.1524) (layer B.Cu) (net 5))
 (segment (start 196.31 119.92) (end 190.5 119.92) (width 0.1524) (layer B.Cu) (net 5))
 (segment (start 188.65 121.77) (end 188.65 121.23) (width 0.1524) (layer B.Cu) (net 5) (status 30))
 (segment (start 204.47 105.41) (end 204.47 108.585) (width 0.1524) (layer B.Cu) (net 7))
 (segment (start 203.2 110.49) (end 203.2 109.855) (width 0.1524) (layer B.Cu) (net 7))
 (segment (start 203.2 109.855) (end 204.47 108.585) (width 0.1524) (layer B.Cu) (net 7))
 (segment (start 203.89 121.77) (end 203.985 121.77) (width 0.1524) (layer B.Cu) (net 7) (status 30))
 (segment (start 203.985 121.77) (end 205.105 120.65) (width 0.1524) (layer B.Cu) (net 7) (status 10))
 (segment (start 203.2 115.57) (end 203.2 110.49) (width 0.1524) (layer B.Cu) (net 7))
 (segment (start 205.105 117.475) (end 203.2 115.57) (width 0.1524) (layer B.Cu) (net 7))
 (segment (start 205.105 120.65) (end 205.105 117.475) (width 0.1524) (layer B.Cu) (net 7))
 (segment (start 204.47 121.19) (end 203.89 121.77) (width 0.1524) (layer B.Cu) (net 7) (status 30))
 (segment (start 203.89 121.77) (end 203.89 121.23) (width 0.1524) (layer B.Cu) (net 7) (status 30))
 (segment (start 207.01 105.41) (end 207.01 108.585) (width 0.1524) (layer B.Cu) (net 8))
 (segment (start 205.74 110.49) (end 205.74 109.855) (width 0.1524) (layer B.Cu) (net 8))
 (segment (start 205.74 109.855) (end 207.01 108.585) (width 0.1524) (layer B.Cu) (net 8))
 (segment (start 205.74 110.49) (end 205.74 123.19) (width 0.1524) (layer B.Cu) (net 8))
 (segment (start 205.74 123.19) (end 210.82 123.19) (width 0.1524) (layer B.Cu) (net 8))
 (segment (start 210.82 123.19) (end 211.51 122.5) (width 0.1524) (layer B.Cu) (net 8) (status 20))
 (segment (start 211.51 122.5) (end 211.51 121.77) (width 0.1524) (layer B.Cu) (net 8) (status 30))
 (segment (start 209.55 105.41) (end 209.55 108.585) (width 0.1524) (layer B.Cu) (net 9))
 (segment (start 210.82 109.855) (end 209.55 108.585) (width 0.1524) (layer B.Cu) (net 9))
 (segment (start 213.36 120.65) (end 212.09 119.38) (width 0.1524) (layer B.Cu) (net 9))
 (segment (start 210.82 109.855) (end 210.82 115.57) (width 0.1524) (layer B.Cu) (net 9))
 (segment (start 212.09 116.84) (end 210.82 115.57) (width 0.1524) (layer B.Cu) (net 9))
 (segment (start 213.36 123.19) (end 218.44 123.19) (width 0.1524) (layer B.Cu) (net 9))
 (segment (start 218.44 123.19) (end 219.13 122.5) (width 0.1524) (layer B.Cu) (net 9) (status 20))
 (segment (start 213.36 120.65) (end 213.36 123.19) (width 0.1524) (layer B.Cu) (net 9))
 (segment (start 212.09 119.38) (end 212.09 116.84) (width 0.1524) (layer B.Cu) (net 9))
 (segment (start 219.13 122.5) (end 219.13 121.77) (width 0.1524) (layer B.Cu) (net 9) (status 30))
 (segment (start 219.71 121.19) (end 219.13 121.77) (width 0.1524) (layer B.Cu) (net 9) (status 30))
 (segment (start 212.09 105.41) (end 212.09 108.585) (width 0.1524) (layer B.Cu) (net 10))
 (segment (start 213.36 109.855) (end 212.09 108.585) (width 0.1524) (layer B.Cu) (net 10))
 (segment (start 219.71 119.38) (end 220.98 120.65) (width 0.1524) (layer B.Cu) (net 10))
 (segment (start 213.36 109.855) (end 213.36 118.11) (width 0.1524) (layer B.Cu) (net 10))
 (segment (start 214.63 119.38) (end 213.36 118.11) (width 0.1524) (layer B.Cu) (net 10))
 (segment (start 219.71 119.38) (end 214.63 119.38) (width 0.1524) (layer B.Cu) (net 10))
 (segment (start 220.98 120.65) (end 220.98 123.19) (width 0.1524) (layer B.Cu) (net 10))
 (segment (start 220.98 123.19) (end 226.06 123.19) (width 0.1524) (layer B.Cu) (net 10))
 (segment (start 226.06 123.19) (end 226.75 122.5) (width 0.1524) (layer B.Cu) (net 10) (status 20))
 (segment (start 226.75 122.5) (end 226.75 121.77) (width 0.1524) (layer B.Cu) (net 10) (status 30))
 (segment (start 227.48 121.77) (end 226.75 121.77) (width 0.1524) (layer B.Cu) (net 10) (status 30))
 (segment (start 217.805 116.205) (end 215.9 114.3) (width 0.1524) (layer B.Cu) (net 11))
 (segment (start 215.9 113.03) (end 215.9 114.3) (width 0.1524) (layer B.Cu) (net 11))
 (segment (start 215.9 109.855) (end 215.9 113.03) (width 0.1524) (layer B.Cu) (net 11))
 (segment (start 215.9 109.855) (end 214.63 108.585) (width 0.1524) (layer B.Cu) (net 11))
 (segment (start 217.805 116.205) (end 219.075 116.205) (width 0.1524) (layer B.Cu) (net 11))
 (segment (start 214.63 105.41) (end 214.63 108.585) (width 0.1524) (layer B.Cu) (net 11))
 (segment (start 222.25 119.38) (end 219.075 116.205) (width 0.1524) (layer B.Cu) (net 11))
 (segment (start 233.68 123.19) (end 234.37 122.5) (width 0.1524) (layer B.Cu) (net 11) (status 20))
 (segment (start 228.6 123.19) (end 233.68 123.19) (width 0.1524) (layer B.Cu) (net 11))
 (segment (start 228.6 120.65) (end 228.6 123.19) (width 0.1524) (layer B.Cu) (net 11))
 (segment (start 227.33 119.38) (end 228.6 120.65) (width 0.1524) (layer B.Cu) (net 11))
 (segment (start 222.25 119.38) (end 227.33 119.38) (width 0.1524) (layer B.Cu) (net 11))
 (segment (start 234.37 122.5) (end 234.37 121.77) (width 0.1524) (layer B.Cu) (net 11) (status 30))
 (segment (start 196.85 113.03) (end 196.85 113.665) (width 0.1524) (layer F.Cu) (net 20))
 (segment (start 195.58 114.935) (end 194.945 114.935) (width 0.1524) (layer F.Cu) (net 20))
 (segment (start 196.85 113.665) (end 195.58 114.935) (width 0.1524) (layer F.Cu) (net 20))
 (segment (start 188.595 116.205) (end 189.865 116.205) (width 0.1524) (layer F.Cu) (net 20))
 (segment (start 189.865 116.205) (end 191.135 114.935) (width 0.1524) (layer F.Cu) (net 20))
 (segment (start 191.135 114.935) (end 194.945 114.935) (width 0.1524) (layer F.Cu) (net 20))
 (segment (start 196.85 111.76) (end 196.85 113.03) (width 0.1524) (layer F.Cu) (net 20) (status 10))
 (segment (start 182.245 116.205) (end 188.595 116.205) (width 0.1524) (layer F.Cu) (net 20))
 (segment (start 180.34 118.11) (end 182.245 116.205) (width 0.1524) (layer F.Cu) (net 20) (status 10))
 (segment (start 199.39 111.76) (end 199.39 113.665) (width 0.1524) (layer F.Cu) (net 21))
 (segment (start 190.5 118.11) (end 187.96 118.11) (width 0.1524) (layer F.Cu) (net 21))
 (segment (start 192.405 116.205) (end 190.5 118.11) (width 0.1524) (layer F.Cu) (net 21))
 (segment (start 196.85 116.205) (end 192.405 116.205) (width 0.1524) (layer F.Cu) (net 21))
 (segment (start 199.39 113.665) (end 196.85 116.205) (width 0.1524) (layer F.Cu) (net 21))
 (segment (start 197.485 118.11) (end 195.58 118.11) (width 0.1524) (layer F.Cu) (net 22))
 (segment (start 201.93 113.665) (end 197.485 118.11) (width 0.1524) (layer F.Cu) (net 22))
 (segment (start 201.93 111.76) (end 201.93 113.665) (width 0.1524) (layer F.Cu) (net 22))
 (segment (start 204.47 111.76) (end 204.47 116.84) (width 0.1524) (layer F.Cu) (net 23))
 (segment (start 204.47 116.84) (end 203.2 118.11) (width 0.1524) (layer F.Cu) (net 23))
 (segment (start 207.01 111.125) (end 207.01 114.3) (width 0.1524) (layer F.Cu) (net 24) (status 10))
 (segment (start 207.01 114.3) (end 210.82 118.11) (width 0.1524) (layer F.Cu) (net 24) (status 20))
 (segment (start 218.44 118.11) (end 217.17 116.84) (width 0.1524) (layer F.Cu) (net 25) (status 10))
 (segment (start 209.55 113.03) (end 209.55 111.125) (width 0.1524) (layer F.Cu) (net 25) (status 20))
 (segment (start 213.36 116.84) (end 209.55 113.03) (width 0.1524) (layer F.Cu) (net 25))
 (segment (start 217.17 116.84) (end 213.36 116.84) (width 0.1524) (layer F.Cu) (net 25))
 (segment (start 212.09 111.125) (end 212.09 113.03) (width 0.1524) (layer F.Cu) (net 26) (status 10))
 (segment (start 223.52 115.57) (end 226.06 118.11) (width 0.1524) (layer F.Cu) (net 26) (status 20))
 (segment (start 214.63 115.57) (end 223.52 115.57) (width 0.1524) (layer F.Cu) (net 26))
 (segment (start 212.09 113.03) (end 214.63 115.57) (width 0.1524) (layer F.Cu) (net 26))
 (segment (start 233.68 118.11) (end 229.87 114.3) (width 0.1524) (layer F.Cu) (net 2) (status 10))
 (segment (start 229.87 114.3) (end 215.9 114.3) (width 0.1524) (layer F.Cu) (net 2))
 (segment (start 214.63 111.125) (end 214.63 113.03) (width 0.1524) (layer F.Cu) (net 2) (status 10))
 (segment (start 214.63 113.03) (end 215.9 114.3) (width 0.1524) (layer F.Cu) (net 2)))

